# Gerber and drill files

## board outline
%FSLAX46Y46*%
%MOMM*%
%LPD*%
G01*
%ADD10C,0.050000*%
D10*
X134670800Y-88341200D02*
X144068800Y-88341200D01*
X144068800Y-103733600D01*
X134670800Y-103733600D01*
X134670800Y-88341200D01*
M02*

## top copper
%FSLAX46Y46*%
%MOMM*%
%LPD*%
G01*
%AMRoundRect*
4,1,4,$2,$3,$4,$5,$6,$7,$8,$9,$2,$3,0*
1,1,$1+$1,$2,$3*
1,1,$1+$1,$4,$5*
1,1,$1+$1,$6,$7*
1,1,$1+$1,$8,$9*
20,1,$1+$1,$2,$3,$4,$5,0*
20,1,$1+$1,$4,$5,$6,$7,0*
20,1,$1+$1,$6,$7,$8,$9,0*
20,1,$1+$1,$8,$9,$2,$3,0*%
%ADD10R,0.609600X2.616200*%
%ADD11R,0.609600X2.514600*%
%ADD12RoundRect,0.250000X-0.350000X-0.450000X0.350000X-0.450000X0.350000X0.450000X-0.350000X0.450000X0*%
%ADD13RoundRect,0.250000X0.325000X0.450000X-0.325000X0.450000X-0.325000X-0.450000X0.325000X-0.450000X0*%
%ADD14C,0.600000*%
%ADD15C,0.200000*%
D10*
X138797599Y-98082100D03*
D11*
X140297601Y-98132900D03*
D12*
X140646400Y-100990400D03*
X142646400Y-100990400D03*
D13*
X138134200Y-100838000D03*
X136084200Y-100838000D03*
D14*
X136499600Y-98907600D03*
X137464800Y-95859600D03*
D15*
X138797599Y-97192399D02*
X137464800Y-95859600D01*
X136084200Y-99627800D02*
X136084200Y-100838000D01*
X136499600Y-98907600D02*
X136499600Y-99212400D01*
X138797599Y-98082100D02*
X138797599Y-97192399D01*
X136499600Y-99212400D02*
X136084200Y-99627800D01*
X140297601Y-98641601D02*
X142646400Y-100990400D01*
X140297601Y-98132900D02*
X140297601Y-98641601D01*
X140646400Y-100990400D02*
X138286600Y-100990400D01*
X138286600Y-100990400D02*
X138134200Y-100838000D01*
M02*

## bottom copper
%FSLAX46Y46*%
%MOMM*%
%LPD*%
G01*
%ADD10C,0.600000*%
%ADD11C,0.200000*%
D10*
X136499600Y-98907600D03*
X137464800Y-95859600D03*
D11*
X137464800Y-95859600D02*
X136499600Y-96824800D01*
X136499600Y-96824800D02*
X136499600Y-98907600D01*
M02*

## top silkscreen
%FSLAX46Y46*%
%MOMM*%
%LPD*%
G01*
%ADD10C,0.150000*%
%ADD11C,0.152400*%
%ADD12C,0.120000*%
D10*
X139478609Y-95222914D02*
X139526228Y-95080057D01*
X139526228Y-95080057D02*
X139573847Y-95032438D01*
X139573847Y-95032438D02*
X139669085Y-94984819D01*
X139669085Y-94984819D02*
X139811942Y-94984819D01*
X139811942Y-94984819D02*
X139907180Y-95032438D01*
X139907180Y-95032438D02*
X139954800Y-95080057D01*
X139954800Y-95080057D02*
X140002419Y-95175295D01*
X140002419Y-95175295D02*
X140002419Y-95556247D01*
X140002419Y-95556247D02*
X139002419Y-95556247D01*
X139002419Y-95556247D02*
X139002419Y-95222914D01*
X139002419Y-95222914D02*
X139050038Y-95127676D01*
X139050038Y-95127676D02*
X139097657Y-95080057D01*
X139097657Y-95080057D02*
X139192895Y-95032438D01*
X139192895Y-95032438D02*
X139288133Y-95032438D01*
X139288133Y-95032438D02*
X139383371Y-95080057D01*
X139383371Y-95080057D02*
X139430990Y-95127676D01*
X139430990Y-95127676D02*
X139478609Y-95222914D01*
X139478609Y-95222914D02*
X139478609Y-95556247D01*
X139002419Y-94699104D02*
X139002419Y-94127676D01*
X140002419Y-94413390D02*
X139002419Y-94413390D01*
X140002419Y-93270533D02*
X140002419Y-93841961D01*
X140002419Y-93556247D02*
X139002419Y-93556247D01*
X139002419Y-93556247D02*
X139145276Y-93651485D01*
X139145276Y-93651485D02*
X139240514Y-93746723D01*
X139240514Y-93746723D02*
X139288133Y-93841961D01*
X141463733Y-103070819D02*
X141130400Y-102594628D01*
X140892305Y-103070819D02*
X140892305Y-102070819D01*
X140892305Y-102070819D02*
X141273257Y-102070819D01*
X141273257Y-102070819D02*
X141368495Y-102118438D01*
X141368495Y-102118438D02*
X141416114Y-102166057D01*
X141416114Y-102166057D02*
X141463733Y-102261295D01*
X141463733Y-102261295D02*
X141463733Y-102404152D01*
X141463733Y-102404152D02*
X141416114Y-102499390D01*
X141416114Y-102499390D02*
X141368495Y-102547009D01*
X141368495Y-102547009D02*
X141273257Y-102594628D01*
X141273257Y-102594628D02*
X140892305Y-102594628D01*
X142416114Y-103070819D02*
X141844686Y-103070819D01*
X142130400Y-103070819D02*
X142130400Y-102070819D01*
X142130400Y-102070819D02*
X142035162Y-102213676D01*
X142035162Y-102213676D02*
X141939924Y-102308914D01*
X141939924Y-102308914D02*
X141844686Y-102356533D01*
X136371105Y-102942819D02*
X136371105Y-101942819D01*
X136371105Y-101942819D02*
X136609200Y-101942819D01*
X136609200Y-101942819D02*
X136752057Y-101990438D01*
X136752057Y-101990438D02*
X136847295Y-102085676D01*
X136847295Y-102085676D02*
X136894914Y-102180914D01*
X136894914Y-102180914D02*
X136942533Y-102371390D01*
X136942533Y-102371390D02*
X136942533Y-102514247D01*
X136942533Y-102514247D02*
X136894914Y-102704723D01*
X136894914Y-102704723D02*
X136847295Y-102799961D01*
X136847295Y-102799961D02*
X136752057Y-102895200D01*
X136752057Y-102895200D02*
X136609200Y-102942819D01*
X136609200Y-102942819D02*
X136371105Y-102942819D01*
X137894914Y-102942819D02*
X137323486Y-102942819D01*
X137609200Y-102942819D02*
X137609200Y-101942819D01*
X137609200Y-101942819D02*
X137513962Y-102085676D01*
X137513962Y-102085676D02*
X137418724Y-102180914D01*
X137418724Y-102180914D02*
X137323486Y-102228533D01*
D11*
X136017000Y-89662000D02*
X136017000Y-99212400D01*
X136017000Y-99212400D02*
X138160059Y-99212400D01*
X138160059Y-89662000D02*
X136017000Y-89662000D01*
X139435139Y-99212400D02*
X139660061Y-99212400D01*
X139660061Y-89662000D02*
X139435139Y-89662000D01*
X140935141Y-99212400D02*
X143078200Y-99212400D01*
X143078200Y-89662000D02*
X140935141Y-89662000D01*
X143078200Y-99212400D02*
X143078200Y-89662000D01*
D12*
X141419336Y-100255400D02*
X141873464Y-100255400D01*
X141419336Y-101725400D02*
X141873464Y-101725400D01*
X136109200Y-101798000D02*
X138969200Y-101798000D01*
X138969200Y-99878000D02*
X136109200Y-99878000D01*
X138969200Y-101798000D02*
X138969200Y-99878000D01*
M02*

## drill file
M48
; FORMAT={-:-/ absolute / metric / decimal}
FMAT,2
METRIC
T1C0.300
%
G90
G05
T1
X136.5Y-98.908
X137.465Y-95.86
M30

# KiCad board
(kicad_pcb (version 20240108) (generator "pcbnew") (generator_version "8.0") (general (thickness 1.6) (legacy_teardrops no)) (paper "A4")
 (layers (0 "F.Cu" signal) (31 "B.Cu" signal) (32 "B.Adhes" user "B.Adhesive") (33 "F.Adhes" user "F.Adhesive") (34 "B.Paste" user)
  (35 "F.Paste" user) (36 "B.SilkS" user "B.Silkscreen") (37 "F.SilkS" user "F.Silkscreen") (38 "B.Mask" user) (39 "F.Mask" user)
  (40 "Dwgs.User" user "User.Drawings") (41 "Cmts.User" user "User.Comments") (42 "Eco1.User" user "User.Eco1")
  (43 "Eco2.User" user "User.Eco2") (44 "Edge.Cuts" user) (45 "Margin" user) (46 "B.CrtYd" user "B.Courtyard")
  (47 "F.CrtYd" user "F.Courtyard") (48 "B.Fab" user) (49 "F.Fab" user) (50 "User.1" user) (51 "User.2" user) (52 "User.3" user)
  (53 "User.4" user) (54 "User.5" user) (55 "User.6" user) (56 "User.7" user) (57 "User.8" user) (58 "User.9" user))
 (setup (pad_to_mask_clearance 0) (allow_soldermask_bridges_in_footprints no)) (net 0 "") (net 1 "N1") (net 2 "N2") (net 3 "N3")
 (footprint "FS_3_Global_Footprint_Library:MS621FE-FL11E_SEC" (layer "F.Cu") (at 139.5476 94.4372 90)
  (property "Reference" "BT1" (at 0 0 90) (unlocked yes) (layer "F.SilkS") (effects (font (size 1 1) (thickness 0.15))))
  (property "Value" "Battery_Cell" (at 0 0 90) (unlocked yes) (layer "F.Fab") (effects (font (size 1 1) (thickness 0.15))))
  (fp_line (start 4.7752 -3.5306) (end -4.7752 -3.5306) (stroke (width 0.1524) (type solid)) (layer "F.SilkS"))
  (fp_line (start -4.7752 -3.5306) (end -4.7752 -1.387541) (stroke (width 0.1524) (type solid)) (layer "F.SilkS"))
  (fp_line (start 4.7752 -1.387541) (end 4.7752 -3.5306) (stroke (width 0.1524) (type solid)) (layer "F.SilkS"))
  (fp_line (start -4.7752 -0.112461) (end -4.7752 0.112461) (stroke (width 0.1524) (type solid)) (layer "F.SilkS"))
  (fp_line (start 4.7752 0.112461) (end 4.7752 -0.112461) (stroke (width 0.1524) (type solid)) (layer "F.SilkS"))
  (fp_line (start -4.7752 1.387541) (end -4.7752 3.5306) (stroke (width 0.1524) (type solid)) (layer "F.SilkS"))
  (fp_line (start 4.7752 3.5306) (end 4.7752 1.387541) (stroke (width 0.1524) (type solid)) (layer "F.SilkS"))
  (fp_line (start -4.7752 3.5306) (end 4.7752 3.5306) (stroke (width 0.1524) (type solid)) (layer "F.SilkS"))
  (pad "1" smd rect (at -3.6449 -0.750001 90) (size 2.6162 0.6096) (layers "F.Cu" "F.Paste" "F.Mask") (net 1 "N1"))
  (pad "2" smd rect (at -3.6957 0.750001 90) (size 2.5146 0.6096) (layers "F.Cu" "F.Paste" "F.Mask") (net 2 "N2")))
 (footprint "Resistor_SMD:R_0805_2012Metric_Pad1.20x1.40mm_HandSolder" (layer "F.Cu") (at 141.6464 100.9904)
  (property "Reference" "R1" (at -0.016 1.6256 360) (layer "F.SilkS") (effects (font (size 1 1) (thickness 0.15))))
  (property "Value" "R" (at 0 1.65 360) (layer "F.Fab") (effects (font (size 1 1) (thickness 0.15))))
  (fp_line (start -0.227064 -0.735) (end 0.227064 -0.735) (stroke (width 0.12) (type solid)) (layer "F.SilkS"))
  (fp_line (start -0.227064 0.735) (end 0.227064 0.735) (stroke (width 0.12) (type solid)) (layer "F.SilkS"))
  (pad "1" smd roundrect (at -1 0) (size 1.2 1.4) (layers "F.Cu" "F.Paste" "F.Mask") (roundrect_rratio 0.208333) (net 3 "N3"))
  (pad "2" smd roundrect (at 1 0) (size 1.2 1.4) (layers "F.Cu" "F.Paste" "F.Mask") (roundrect_rratio 0.208333) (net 2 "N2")))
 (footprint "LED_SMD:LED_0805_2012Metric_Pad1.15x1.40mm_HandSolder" (layer "F.Cu") (at 137.1092 100.838 180)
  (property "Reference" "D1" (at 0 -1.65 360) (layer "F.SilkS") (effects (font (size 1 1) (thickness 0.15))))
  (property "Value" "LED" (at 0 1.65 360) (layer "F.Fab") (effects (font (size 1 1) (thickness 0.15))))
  (fp_line (start 1 -0.96) (end -1.86 -0.96) (stroke (width 0.12) (type solid)) (layer "F.SilkS"))
  (fp_line (start -1.86 0.96) (end 1 0.96) (stroke (width 0.12) (type solid)) (layer "F.SilkS"))
  (fp_line (start -1.86 -0.96) (end -1.86 0.96) (stroke (width 0.12) (type solid)) (layer "F.SilkS"))
  (pad "1" smd roundrect (at -1.025 0 180) (size 1.15 1.4) (layers "F.Cu" "F.Paste" "F.Mask") (roundrect_rratio 0.217391) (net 3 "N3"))
  (pad "2" smd roundrect (at 1.025 0 180) (size 1.15 1.4) (layers "F.Cu" "F.Paste" "F.Mask") (roundrect_rratio 0.217391) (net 1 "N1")))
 (gr_rect (start 134.6708 88.3412) (end 144.0688 103.7336) (stroke (width 0.05) (type default)) (fill none) (layer "Edge.Cuts"))
 (segment (start 138.797599 97.192399) (end 137.4648 95.8596) (width 0.2) (layer "F.Cu") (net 1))
 (segment (start 136.0842 99.6278) (end 136.0842 100.838) (width 0.2) (layer "F.Cu") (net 1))
 (segment (start 136.4996 98.9076) (end 136.4996 99.2124) (width 0.2) (layer "F.Cu") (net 1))
 (segment (start 138.797599 98.0821) (end 138.797599 97.192399) (width 0.2) (layer "F.Cu") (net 1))
 (segment (start 136.4996 99.2124) (end 136.0842 99.6278) (width 0.2) (layer "F.Cu") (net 1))
 (via (at 136.4996 98.9076) (size 0.6) (drill 0.3) (layers "F.Cu" "B.Cu") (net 1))
 (via (at 137.4648 95.8596) (size 0.6) (drill 0.3) (layers "F.Cu" "B.Cu") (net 1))
 (segment (start 137.4648 95.8596) (end 136.4996 96.8248) (width 0.2) (layer "B.Cu") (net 1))
 (segment (start 136.4996 96.8248) (end 136.4996 98.9076) (width 0.2) (layer "B.Cu") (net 1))
 (segment (start 140.297601 98.641601) (end 142.6464 100.9904) (width 0.2) (layer "F.Cu") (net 2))
 (segment (start 140.297601 98.1329) (end 140.297601 98.641601) (width 0.2) (layer "F.Cu") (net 2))
 (segment (start 140.6464 100.9904) (end 138.2866 100.9904) (width 0.2) (layer "F.Cu") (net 3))
 (segment (start 138.2866 100.9904) (end 138.1342 100.838) (width 0.2) (layer "F.Cu") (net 3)))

